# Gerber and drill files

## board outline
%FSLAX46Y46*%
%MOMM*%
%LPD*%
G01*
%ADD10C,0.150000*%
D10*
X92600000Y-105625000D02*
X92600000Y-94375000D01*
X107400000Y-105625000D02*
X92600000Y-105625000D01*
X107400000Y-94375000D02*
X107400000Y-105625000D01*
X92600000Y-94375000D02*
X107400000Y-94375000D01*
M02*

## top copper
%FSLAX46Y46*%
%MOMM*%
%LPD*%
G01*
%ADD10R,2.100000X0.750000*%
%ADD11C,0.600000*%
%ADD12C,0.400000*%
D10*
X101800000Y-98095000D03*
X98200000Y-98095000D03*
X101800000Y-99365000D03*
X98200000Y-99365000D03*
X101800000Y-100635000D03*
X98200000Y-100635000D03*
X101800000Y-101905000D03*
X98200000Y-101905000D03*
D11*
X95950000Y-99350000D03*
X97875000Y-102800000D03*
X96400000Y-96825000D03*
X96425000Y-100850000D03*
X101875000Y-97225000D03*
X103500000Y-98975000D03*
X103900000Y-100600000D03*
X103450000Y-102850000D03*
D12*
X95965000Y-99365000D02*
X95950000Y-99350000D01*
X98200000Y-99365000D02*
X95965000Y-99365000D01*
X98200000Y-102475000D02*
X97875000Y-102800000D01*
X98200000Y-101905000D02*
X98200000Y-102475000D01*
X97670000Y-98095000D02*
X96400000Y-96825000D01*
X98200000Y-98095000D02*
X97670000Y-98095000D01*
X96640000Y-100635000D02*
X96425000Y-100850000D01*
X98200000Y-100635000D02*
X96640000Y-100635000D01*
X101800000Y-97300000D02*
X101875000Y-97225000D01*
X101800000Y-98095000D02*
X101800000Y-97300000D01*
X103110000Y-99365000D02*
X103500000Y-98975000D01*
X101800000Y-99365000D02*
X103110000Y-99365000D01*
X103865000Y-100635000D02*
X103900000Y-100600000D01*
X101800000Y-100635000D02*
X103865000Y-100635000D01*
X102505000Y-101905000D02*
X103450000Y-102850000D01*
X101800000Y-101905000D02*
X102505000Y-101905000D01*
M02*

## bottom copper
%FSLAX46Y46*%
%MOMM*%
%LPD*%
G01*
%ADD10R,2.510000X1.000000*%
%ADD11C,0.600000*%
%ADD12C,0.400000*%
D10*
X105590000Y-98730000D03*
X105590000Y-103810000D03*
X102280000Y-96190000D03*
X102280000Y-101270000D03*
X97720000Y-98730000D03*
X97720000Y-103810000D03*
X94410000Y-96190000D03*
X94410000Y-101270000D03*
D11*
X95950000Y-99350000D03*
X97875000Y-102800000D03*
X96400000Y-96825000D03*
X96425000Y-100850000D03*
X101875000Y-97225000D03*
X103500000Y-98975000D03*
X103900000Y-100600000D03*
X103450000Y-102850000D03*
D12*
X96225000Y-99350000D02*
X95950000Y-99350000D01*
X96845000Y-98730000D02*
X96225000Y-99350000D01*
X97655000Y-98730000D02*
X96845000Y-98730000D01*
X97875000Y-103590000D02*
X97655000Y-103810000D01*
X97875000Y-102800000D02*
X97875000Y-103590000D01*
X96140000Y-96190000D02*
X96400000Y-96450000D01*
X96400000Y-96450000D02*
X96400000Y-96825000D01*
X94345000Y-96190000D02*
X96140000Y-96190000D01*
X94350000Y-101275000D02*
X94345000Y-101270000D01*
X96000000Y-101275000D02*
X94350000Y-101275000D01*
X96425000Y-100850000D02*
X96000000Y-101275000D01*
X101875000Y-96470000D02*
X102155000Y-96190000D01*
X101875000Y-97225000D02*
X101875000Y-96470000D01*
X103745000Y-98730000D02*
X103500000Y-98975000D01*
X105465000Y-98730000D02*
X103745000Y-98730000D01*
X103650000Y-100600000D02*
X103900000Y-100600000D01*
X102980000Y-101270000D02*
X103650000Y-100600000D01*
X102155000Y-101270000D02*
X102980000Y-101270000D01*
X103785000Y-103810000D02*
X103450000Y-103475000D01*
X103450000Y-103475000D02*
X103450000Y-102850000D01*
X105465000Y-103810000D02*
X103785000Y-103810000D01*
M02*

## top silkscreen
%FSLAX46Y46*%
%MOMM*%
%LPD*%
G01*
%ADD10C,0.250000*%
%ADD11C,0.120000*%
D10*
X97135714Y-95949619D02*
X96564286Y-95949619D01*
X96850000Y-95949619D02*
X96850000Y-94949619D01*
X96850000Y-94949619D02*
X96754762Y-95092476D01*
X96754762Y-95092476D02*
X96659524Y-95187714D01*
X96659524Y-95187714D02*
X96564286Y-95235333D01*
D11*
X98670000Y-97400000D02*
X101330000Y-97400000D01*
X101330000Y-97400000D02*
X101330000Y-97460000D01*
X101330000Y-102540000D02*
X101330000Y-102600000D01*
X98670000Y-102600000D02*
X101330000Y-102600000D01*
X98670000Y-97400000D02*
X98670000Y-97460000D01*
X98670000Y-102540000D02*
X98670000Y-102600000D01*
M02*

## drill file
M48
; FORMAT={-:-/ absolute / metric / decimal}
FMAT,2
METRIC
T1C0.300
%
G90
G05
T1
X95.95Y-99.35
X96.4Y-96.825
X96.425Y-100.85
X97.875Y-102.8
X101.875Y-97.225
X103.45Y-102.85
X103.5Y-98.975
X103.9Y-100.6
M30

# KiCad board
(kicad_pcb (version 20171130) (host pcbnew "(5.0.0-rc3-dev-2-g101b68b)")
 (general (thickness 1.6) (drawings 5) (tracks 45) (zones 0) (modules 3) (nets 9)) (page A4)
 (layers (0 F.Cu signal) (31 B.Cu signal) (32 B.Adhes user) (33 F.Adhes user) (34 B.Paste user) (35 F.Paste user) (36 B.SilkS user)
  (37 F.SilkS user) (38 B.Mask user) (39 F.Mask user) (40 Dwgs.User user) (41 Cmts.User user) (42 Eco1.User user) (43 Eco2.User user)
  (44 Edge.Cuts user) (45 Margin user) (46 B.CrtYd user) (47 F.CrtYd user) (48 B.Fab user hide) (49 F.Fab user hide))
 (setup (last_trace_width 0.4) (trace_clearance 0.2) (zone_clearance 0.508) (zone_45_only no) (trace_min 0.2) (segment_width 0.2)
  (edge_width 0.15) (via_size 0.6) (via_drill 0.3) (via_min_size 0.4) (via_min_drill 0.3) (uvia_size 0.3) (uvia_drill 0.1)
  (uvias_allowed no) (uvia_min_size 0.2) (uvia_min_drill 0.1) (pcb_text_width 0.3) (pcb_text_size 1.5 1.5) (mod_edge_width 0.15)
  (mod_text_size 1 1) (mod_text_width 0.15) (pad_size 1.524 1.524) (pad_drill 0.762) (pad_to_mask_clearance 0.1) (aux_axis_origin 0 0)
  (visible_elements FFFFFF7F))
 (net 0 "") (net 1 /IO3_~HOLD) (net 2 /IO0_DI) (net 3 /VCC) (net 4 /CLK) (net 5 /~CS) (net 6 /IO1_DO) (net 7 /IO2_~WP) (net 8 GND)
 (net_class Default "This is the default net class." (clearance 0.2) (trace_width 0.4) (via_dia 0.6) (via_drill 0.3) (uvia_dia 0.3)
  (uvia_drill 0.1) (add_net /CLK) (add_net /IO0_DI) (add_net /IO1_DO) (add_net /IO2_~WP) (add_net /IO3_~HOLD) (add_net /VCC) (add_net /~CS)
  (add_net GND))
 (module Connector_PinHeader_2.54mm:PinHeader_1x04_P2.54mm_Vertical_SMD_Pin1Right (layer B.Cu) (at 103.935 100)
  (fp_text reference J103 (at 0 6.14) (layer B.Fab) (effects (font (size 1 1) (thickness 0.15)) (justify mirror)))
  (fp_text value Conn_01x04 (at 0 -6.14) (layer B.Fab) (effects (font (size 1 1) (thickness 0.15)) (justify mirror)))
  (pad 3 smd rect (at 1.655 -1.27) (size 2.51 1) (layers B.Cu B.Paste B.Mask) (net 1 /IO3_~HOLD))
  (pad 1 smd rect (at 1.655 3.81) (size 2.51 1) (layers B.Cu B.Paste B.Mask) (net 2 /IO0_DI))
  (pad 4 smd rect (at -1.655 -3.81) (size 2.51 1) (layers B.Cu B.Paste B.Mask) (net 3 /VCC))
  (pad 2 smd rect (at -1.655 1.27) (size 2.51 1) (layers B.Cu B.Paste B.Mask) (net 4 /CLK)))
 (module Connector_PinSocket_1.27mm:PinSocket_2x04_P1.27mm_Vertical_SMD (layer F.Cu) (at 100 100)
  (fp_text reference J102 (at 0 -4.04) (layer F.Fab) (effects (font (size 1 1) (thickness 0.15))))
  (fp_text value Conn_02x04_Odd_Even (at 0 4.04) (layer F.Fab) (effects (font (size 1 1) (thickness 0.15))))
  (fp_line (start -1.33 -2.6) (end 1.33 -2.6) (layer F.SilkS) (width 0.12))
  (fp_line (start 1.33 -2.6) (end 1.33 -2.54) (layer F.SilkS) (width 0.12))
  (fp_line (start 1.33 2.54) (end 1.33 2.6) (layer F.SilkS) (width 0.12))
  (fp_line (start -1.33 2.6) (end 1.33 2.6) (layer F.SilkS) (width 0.12))
  (fp_line (start -1.33 -2.6) (end -1.33 -2.54) (layer F.SilkS) (width 0.12))
  (fp_line (start -1.33 2.54) (end -1.33 2.6) (layer F.SilkS) (width 0.12))
  (pad 1 smd rect (at 1.8 -1.905) (size 2.1 0.75) (layers F.Cu F.Paste F.Mask) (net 3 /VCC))
  (pad 2 smd rect (at -1.8 -1.905) (size 2.1 0.75) (layers F.Cu F.Paste F.Mask) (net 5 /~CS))
  (pad 3 smd rect (at 1.8 -0.635) (size 2.1 0.75) (layers F.Cu F.Paste F.Mask) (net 1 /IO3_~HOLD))
  (pad 4 smd rect (at -1.8 -0.635) (size 2.1 0.75) (layers F.Cu F.Paste F.Mask) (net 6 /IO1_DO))
  (pad 5 smd rect (at 1.8 0.635) (size 2.1 0.75) (layers F.Cu F.Paste F.Mask) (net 4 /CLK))
  (pad 6 smd rect (at -1.8 0.635) (size 2.1 0.75) (layers F.Cu F.Paste F.Mask) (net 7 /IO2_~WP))
  (pad 7 smd rect (at 1.8 1.905) (size 2.1 0.75) (layers F.Cu F.Paste F.Mask) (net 2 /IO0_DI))
  (pad 8 smd rect (at -1.8 1.905) (size 2.1 0.75) (layers F.Cu F.Paste F.Mask) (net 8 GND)))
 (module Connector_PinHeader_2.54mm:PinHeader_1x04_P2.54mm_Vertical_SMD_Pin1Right (layer B.Cu) (at 96.065 100 180)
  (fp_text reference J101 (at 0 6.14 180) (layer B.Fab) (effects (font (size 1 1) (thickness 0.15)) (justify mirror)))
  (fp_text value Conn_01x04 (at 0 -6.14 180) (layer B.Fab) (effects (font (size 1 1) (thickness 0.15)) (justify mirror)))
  (pad 2 smd rect (at -1.655 1.27 180) (size 2.51 1) (layers B.Cu B.Paste B.Mask) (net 6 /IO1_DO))
  (pad 4 smd rect (at -1.655 -3.81 180) (size 2.51 1) (layers B.Cu B.Paste B.Mask) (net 8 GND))
  (pad 1 smd rect (at 1.655 3.81 180) (size 2.51 1) (layers B.Cu B.Paste B.Mask) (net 5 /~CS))
  (pad 3 smd rect (at 1.655 -1.27 180) (size 2.51 1) (layers B.Cu B.Paste B.Mask) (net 7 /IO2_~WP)))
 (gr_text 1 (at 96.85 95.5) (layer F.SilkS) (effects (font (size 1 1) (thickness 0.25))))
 (gr_line (start 92.6 105.625) (end 92.6 94.375) (layer Edge.Cuts) (width 0.15))
 (gr_line (start 107.4 105.625) (end 92.6 105.625) (layer Edge.Cuts) (width 0.15))
 (gr_line (start 107.4 94.375) (end 107.4 105.625) (layer Edge.Cuts) (width 0.15))
 (gr_line (start 92.6 94.375) (end 107.4 94.375) (layer Edge.Cuts) (width 0.15))
 (via (at 95.95 99.35) (size 0.6) (drill 0.3) (layers F.Cu B.Cu) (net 6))
 (segment (start 95.965 99.365) (end 95.95 99.35) (width 0.4) (layer F.Cu) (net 6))
 (segment (start 98.2 99.365) (end 95.965 99.365) (width 0.4) (layer F.Cu) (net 6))
 (segment (start 96.225 99.35) (end 95.95 99.35) (width 0.4) (layer B.Cu) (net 6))
 (segment (start 96.845 98.73) (end 96.225 99.35) (width 0.4) (layer B.Cu) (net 6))
 (segment (start 97.655 98.73) (end 96.845 98.73) (width 0.4) (layer B.Cu) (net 6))
 (via (at 97.875 102.8) (size 0.6) (drill 0.3) (layers F.Cu B.Cu) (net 8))
 (segment (start 98.2 102.475) (end 97.875 102.8) (width 0.4) (layer F.Cu) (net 8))
 (segment (start 98.2 101.905) (end 98.2 102.475) (width 0.4) (layer F.Cu) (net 8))
 (segment (start 97.875 103.59) (end 97.655 103.81) (width 0.4) (layer B.Cu) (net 8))
 (segment (start 97.875 102.8) (end 97.875 103.59) (width 0.4) (layer B.Cu) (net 8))
 (segment (start 97.67 98.095) (end 96.4 96.825) (width 0.4) (layer F.Cu) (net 5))
 (via (at 96.4 96.825) (size 0.6) (drill 0.3) (layers F.Cu B.Cu) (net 5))
 (segment (start 98.2 98.095) (end 97.67 98.095) (width 0.4) (layer F.Cu) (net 5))
 (segment (start 96.14 96.19) (end 96.4 96.45) (width 0.4) (layer B.Cu) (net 5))
 (segment (start 96.4 96.45) (end 96.4 96.825) (width 0.4) (layer B.Cu) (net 5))
 (segment (start 94.345 96.19) (end 96.14 96.19) (width 0.4) (layer B.Cu) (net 5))
 (via (at 96.425 100.85) (size 0.6) (drill 0.3) (layers F.Cu B.Cu) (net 7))
 (segment (start 96.64 100.635) (end 96.425 100.85) (width 0.4) (layer F.Cu) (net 7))
 (segment (start 98.2 100.635) (end 96.64 100.635) (width 0.4) (layer F.Cu) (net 7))
 (segment (start 94.35 101.275) (end 94.345 101.27) (width 0.4) (layer B.Cu) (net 7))
 (segment (start 96 101.275) (end 94.35 101.275) (width 0.4) (layer B.Cu) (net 7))
 (segment (start 96.425 100.85) (end 96 101.275) (width 0.4) (layer B.Cu) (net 7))
 (via (at 101.875 97.225) (size 0.6) (drill 0.3) (layers F.Cu B.Cu) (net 3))
 (segment (start 101.8 97.3) (end 101.875 97.225) (width 0.4) (layer F.Cu) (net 3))
 (segment (start 101.8 98.095) (end 101.8 97.3) (width 0.4) (layer F.Cu) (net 3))
 (segment (start 101.875 96.47) (end 102.155 96.19) (width 0.4) (layer B.Cu) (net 3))
 (segment (start 101.875 97.225) (end 101.875 96.47) (width 0.4) (layer B.Cu) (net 3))
 (via (at 103.5 98.975) (size 0.6) (drill 0.3) (layers F.Cu B.Cu) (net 1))
 (segment (start 103.11 99.365) (end 103.5 98.975) (width 0.4) (layer F.Cu) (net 1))
 (segment (start 101.8 99.365) (end 103.11 99.365) (width 0.4) (layer F.Cu) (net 1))
 (segment (start 103.745 98.73) (end 103.5 98.975) (width 0.4) (layer B.Cu) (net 1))
 (segment (start 105.465 98.73) (end 103.745 98.73) (width 0.4) (layer B.Cu) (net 1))
 (segment (start 103.865 100.635) (end 103.9 100.6) (width 0.4) (layer F.Cu) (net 4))
 (segment (start 101.8 100.635) (end 103.865 100.635) (width 0.4) (layer F.Cu) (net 4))
 (via (at 103.9 100.6) (size 0.6) (drill 0.3) (layers F.Cu B.Cu) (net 4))
 (segment (start 103.65 100.6) (end 103.9 100.6) (width 0.4) (layer B.Cu) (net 4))
 (segment (start 102.98 101.27) (end 103.65 100.6) (width 0.4) (layer B.Cu) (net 4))
 (segment (start 102.155 101.27) (end 102.98 101.27) (width 0.4) (layer B.Cu) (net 4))
 (via (at 103.45 102.85) (size 0.6) (drill 0.3) (layers F.Cu B.Cu) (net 2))
 (segment (start 102.505 101.905) (end 103.45 102.85) (width 0.4) (layer F.Cu) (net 2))
 (segment (start 101.8 101.905) (end 102.505 101.905) (width 0.4) (layer F.Cu) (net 2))
 (segment (start 103.785 103.81) (end 103.45 103.475) (width 0.4) (layer B.Cu) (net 2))
 (segment (start 103.45 103.475) (end 103.45 102.85) (width 0.4) (layer B.Cu) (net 2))
 (segment (start 105.465 103.81) (end 103.785 103.81) (width 0.4) (layer B.Cu) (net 2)))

